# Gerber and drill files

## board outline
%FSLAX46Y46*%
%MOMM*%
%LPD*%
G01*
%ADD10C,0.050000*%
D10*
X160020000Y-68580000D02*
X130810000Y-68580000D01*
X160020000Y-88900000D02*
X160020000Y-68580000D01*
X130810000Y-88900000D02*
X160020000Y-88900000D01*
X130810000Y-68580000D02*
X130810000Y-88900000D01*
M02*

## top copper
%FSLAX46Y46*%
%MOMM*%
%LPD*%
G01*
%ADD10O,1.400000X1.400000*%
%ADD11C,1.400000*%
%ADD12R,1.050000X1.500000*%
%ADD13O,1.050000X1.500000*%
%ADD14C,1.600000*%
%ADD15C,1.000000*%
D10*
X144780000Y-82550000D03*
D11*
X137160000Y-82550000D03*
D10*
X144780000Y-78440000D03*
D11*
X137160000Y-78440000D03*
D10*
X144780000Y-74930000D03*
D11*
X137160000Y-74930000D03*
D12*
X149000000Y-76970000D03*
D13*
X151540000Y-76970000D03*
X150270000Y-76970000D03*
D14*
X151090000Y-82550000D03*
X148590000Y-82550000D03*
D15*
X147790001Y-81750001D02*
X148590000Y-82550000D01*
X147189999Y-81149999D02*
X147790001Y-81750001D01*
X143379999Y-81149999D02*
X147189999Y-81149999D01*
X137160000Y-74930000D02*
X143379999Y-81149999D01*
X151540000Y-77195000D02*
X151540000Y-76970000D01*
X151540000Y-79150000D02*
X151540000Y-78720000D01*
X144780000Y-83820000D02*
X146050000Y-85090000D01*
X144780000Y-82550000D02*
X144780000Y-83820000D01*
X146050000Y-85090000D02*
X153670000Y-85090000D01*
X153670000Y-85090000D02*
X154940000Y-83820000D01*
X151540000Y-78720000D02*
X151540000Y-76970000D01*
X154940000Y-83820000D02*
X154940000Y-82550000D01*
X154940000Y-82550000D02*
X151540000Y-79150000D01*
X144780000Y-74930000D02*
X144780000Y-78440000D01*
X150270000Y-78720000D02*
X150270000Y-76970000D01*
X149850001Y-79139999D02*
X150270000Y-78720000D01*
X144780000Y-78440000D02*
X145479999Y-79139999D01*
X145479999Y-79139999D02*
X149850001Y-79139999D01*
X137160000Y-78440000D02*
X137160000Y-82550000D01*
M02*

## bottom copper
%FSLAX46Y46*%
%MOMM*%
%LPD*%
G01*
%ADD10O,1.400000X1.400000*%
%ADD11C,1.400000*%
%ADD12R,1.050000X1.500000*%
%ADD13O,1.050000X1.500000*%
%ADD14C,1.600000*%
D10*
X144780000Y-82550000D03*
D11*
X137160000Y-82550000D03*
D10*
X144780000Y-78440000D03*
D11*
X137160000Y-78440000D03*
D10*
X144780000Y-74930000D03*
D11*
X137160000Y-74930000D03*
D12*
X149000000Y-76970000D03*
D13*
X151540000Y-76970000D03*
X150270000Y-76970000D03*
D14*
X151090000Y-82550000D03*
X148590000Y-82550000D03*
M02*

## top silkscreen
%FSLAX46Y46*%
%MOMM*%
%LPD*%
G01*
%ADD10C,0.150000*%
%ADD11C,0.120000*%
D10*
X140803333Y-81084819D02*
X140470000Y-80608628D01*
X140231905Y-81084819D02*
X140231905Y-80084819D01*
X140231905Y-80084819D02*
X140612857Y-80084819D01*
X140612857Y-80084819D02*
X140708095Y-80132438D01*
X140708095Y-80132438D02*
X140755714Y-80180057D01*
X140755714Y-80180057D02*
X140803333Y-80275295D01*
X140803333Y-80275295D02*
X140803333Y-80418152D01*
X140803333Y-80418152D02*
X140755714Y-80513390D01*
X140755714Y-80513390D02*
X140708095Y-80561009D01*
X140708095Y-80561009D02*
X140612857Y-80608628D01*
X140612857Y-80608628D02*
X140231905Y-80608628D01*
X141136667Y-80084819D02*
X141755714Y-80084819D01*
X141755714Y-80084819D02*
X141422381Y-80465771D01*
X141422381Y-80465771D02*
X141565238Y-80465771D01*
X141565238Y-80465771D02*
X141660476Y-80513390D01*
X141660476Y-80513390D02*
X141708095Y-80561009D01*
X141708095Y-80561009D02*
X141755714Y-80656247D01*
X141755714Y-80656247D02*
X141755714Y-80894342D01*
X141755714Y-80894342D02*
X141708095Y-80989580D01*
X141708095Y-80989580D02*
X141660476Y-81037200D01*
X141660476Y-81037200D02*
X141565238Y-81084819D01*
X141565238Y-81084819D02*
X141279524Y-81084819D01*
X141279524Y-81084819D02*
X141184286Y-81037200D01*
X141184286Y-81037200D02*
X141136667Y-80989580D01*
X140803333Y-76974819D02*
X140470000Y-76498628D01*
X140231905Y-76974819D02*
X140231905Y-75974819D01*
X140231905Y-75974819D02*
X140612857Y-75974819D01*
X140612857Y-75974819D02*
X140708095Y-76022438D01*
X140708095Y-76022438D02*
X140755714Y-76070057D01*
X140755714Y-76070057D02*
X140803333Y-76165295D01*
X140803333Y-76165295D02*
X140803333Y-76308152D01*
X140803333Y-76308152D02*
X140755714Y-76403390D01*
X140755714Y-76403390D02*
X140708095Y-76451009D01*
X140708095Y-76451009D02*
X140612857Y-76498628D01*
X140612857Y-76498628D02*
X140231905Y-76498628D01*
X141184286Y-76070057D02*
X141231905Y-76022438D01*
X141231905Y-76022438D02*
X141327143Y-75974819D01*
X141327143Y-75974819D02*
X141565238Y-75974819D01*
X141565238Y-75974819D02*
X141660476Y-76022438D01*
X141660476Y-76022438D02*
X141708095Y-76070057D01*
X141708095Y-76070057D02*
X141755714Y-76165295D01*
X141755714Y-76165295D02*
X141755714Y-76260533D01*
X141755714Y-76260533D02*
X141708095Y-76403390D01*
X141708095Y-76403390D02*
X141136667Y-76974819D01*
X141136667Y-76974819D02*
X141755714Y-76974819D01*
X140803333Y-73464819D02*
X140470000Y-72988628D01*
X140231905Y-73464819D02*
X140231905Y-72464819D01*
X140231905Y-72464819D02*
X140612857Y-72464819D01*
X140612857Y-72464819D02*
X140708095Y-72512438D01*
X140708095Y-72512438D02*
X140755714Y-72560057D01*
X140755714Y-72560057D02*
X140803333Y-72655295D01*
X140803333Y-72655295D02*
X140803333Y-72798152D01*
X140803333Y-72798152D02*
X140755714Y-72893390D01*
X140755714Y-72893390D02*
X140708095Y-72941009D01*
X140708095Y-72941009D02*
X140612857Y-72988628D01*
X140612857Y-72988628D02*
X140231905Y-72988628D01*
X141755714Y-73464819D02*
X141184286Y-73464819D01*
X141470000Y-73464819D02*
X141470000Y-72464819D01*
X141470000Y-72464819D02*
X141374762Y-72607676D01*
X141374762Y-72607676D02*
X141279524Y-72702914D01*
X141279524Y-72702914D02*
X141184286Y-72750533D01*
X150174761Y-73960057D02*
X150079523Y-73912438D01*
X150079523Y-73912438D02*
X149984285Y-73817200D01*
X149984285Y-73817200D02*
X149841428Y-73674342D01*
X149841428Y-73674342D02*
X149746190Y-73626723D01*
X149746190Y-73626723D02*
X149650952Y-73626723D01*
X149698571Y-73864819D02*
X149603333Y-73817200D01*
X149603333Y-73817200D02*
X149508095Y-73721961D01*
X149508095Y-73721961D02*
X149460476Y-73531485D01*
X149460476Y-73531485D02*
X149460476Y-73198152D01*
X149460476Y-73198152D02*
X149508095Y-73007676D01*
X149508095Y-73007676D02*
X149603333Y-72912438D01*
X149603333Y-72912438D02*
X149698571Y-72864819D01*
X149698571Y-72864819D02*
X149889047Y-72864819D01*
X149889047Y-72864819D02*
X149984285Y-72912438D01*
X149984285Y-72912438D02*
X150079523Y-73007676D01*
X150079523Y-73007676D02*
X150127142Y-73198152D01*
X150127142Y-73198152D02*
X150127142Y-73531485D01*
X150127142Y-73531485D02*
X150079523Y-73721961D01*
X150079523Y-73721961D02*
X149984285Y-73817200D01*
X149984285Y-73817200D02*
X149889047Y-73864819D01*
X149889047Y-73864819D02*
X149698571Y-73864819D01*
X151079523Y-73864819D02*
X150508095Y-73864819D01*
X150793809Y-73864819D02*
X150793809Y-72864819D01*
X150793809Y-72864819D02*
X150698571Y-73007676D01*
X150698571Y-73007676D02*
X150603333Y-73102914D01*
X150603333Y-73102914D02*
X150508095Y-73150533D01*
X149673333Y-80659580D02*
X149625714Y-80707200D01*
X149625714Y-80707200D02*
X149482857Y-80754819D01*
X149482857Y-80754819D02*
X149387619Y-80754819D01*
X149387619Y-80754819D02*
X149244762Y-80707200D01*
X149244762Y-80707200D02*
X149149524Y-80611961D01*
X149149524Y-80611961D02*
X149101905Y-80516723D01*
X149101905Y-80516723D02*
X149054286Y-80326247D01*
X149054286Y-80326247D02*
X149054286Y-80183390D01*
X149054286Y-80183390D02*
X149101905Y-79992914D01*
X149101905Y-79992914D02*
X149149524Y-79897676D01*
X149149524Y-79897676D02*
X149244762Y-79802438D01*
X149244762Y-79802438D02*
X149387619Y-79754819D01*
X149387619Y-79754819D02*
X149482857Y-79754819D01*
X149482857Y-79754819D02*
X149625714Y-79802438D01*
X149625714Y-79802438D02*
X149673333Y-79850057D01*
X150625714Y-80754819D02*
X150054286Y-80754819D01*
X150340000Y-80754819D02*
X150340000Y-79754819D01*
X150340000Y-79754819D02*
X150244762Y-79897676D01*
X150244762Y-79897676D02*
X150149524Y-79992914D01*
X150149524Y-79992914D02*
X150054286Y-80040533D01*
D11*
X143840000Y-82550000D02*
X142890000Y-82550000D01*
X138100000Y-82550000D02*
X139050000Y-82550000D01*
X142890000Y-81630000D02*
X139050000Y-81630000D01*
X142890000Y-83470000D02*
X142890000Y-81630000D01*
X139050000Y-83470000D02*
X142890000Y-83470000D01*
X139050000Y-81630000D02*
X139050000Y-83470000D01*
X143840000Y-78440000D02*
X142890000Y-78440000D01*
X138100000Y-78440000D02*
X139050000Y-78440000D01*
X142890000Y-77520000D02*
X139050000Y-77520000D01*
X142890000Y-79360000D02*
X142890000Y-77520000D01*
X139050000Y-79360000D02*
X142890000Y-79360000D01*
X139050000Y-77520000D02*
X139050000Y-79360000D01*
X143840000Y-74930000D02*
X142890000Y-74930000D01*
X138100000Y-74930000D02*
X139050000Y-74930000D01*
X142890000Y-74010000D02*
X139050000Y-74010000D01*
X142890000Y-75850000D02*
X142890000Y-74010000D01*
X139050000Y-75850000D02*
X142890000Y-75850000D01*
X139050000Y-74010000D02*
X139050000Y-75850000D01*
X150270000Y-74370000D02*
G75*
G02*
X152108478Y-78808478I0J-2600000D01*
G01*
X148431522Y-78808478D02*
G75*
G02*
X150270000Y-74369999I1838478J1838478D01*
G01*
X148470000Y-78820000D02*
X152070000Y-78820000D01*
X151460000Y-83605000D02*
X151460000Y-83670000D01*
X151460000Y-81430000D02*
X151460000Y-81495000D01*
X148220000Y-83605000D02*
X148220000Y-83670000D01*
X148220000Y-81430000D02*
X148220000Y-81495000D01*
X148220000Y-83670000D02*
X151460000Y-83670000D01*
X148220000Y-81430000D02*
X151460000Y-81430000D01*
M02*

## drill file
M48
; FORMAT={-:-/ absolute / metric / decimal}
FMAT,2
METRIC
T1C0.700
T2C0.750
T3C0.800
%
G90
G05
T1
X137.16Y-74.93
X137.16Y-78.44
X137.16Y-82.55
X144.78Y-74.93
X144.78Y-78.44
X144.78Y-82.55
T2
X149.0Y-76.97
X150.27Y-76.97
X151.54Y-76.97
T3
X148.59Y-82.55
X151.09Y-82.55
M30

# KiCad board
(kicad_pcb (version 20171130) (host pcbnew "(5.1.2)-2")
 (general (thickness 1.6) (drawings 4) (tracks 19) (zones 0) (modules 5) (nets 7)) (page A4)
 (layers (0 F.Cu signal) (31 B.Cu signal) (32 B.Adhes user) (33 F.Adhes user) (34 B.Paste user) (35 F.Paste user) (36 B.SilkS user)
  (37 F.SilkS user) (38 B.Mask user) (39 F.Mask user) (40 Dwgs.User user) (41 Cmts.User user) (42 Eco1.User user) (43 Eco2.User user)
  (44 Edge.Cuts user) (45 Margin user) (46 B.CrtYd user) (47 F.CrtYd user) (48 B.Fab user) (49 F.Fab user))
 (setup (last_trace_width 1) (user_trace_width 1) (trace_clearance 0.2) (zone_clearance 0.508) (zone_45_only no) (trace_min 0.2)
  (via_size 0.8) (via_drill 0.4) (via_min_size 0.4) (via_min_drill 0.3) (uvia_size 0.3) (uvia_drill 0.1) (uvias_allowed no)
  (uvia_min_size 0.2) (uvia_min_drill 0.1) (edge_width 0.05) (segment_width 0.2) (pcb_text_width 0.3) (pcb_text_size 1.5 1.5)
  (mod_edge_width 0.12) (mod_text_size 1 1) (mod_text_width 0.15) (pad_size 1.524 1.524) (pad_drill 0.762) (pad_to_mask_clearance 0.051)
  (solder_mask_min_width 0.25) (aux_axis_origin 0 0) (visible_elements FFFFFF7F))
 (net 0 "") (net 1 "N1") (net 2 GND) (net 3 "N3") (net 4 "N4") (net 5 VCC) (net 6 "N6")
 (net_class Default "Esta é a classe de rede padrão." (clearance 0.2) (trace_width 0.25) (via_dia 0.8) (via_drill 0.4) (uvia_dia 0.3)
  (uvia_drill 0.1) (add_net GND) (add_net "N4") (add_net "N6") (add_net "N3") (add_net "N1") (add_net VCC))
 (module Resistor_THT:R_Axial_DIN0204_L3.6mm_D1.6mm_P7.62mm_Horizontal (layer F.Cu) (at 137.16 82.55)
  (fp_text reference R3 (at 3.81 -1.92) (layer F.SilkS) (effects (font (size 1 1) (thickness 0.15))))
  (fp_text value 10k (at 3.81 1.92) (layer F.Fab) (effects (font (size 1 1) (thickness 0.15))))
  (fp_line (start 6.68 0) (end 5.73 0) (layer F.SilkS) (width 0.12))
  (fp_line (start 0.94 0) (end 1.89 0) (layer F.SilkS) (width 0.12))
  (fp_line (start 5.73 -0.92) (end 1.89 -0.92) (layer F.SilkS) (width 0.12))
  (fp_line (start 5.73 0.92) (end 5.73 -0.92) (layer F.SilkS) (width 0.12))
  (fp_line (start 1.89 0.92) (end 5.73 0.92) (layer F.SilkS) (width 0.12))
  (fp_line (start 1.89 -0.92) (end 1.89 0.92) (layer F.SilkS) (width 0.12))
  (pad 2 thru_hole oval (at 7.62 0) (size 1.4 1.4) (drill 0.7) (layers *.Cu *.Mask) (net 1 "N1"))
  (pad 1 thru_hole circle (at 0 0) (size 1.4 1.4) (drill 0.7) (layers *.Cu *.Mask) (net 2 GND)))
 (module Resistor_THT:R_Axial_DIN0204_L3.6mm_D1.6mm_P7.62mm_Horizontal (layer F.Cu) (at 137.16 78.44)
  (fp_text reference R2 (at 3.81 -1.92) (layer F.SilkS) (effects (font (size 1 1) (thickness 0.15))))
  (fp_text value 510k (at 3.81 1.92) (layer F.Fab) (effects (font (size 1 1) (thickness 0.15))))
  (fp_line (start 6.68 0) (end 5.73 0) (layer F.SilkS) (width 0.12))
  (fp_line (start 0.94 0) (end 1.89 0) (layer F.SilkS) (width 0.12))
  (fp_line (start 5.73 -0.92) (end 1.89 -0.92) (layer F.SilkS) (width 0.12))
  (fp_line (start 5.73 0.92) (end 5.73 -0.92) (layer F.SilkS) (width 0.12))
  (fp_line (start 1.89 0.92) (end 5.73 0.92) (layer F.SilkS) (width 0.12))
  (fp_line (start 1.89 -0.92) (end 1.89 0.92) (layer F.SilkS) (width 0.12))
  (pad 2 thru_hole oval (at 7.62 0) (size 1.4 1.4) (drill 0.7) (layers *.Cu *.Mask) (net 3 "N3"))
  (pad 1 thru_hole circle (at 0 0) (size 1.4 1.4) (drill 0.7) (layers *.Cu *.Mask) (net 2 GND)))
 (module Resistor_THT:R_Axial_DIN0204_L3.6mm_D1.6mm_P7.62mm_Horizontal (layer F.Cu) (at 137.16 74.93)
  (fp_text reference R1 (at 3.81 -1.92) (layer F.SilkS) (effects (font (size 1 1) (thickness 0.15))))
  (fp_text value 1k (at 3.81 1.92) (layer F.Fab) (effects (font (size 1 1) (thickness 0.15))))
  (fp_line (start 6.68 0) (end 5.73 0) (layer F.SilkS) (width 0.12))
  (fp_line (start 0.94 0) (end 1.89 0) (layer F.SilkS) (width 0.12))
  (fp_line (start 5.73 -0.92) (end 1.89 -0.92) (layer F.SilkS) (width 0.12))
  (fp_line (start 5.73 0.92) (end 5.73 -0.92) (layer F.SilkS) (width 0.12))
  (fp_line (start 1.89 0.92) (end 5.73 0.92) (layer F.SilkS) (width 0.12))
  (fp_line (start 1.89 -0.92) (end 1.89 0.92) (layer F.SilkS) (width 0.12))
  (pad 2 thru_hole oval (at 7.62 0) (size 1.4 1.4) (drill 0.7) (layers *.Cu *.Mask) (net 3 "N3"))
  (pad 1 thru_hole circle (at 0 0) (size 1.4 1.4) (drill 0.7) (layers *.Cu *.Mask) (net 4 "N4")))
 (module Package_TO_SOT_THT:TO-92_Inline (layer F.Cu) (at 149 76.97)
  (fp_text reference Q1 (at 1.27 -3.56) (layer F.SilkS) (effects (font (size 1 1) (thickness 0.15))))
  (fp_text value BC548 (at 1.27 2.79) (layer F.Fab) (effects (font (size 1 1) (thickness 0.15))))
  (fp_arc (start 1.27 0) (end 1.27 -2.6) (angle 135) (layer F.SilkS) (width 0.12))
  (fp_arc (start 1.27 0) (end 1.27 -2.6) (angle -135) (layer F.SilkS) (width 0.12))
  (fp_line (start -0.53 1.85) (end 3.07 1.85) (layer F.SilkS) (width 0.12))
  (pad 1 thru_hole rect (at 0 0) (size 1.05 1.5) (drill 0.75) (layers *.Cu *.Mask) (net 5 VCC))
  (pad 3 thru_hole oval (at 2.54 0) (size 1.05 1.5) (drill 0.75) (layers *.Cu *.Mask) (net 1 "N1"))
  (pad 2 thru_hole oval (at 1.27 0) (size 1.05 1.5) (drill 0.75) (layers *.Cu *.Mask) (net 3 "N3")))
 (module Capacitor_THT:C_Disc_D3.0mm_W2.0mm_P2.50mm (layer F.Cu) (at 148.59 82.55)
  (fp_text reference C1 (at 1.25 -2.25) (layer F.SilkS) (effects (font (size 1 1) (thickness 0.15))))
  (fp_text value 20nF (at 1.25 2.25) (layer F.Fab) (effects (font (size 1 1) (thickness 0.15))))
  (fp_line (start 2.87 1.055) (end 2.87 1.12) (layer F.SilkS) (width 0.12))
  (fp_line (start 2.87 -1.12) (end 2.87 -1.055) (layer F.SilkS) (width 0.12))
  (fp_line (start -0.37 1.055) (end -0.37 1.12) (layer F.SilkS) (width 0.12))
  (fp_line (start -0.37 -1.12) (end -0.37 -1.055) (layer F.SilkS) (width 0.12))
  (fp_line (start -0.37 1.12) (end 2.87 1.12) (layer F.SilkS) (width 0.12))
  (fp_line (start -0.37 -1.12) (end 2.87 -1.12) (layer F.SilkS) (width 0.12))
  (pad 2 thru_hole circle (at 2.5 0) (size 1.6 1.6) (drill 0.8) (layers *.Cu *.Mask) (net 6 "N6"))
  (pad 1 thru_hole circle (at 0 0) (size 1.6 1.6) (drill 0.8) (layers *.Cu *.Mask) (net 4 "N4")))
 (gr_line (start 160.02 68.58) (end 130.81 68.58) (layer Edge.Cuts) (width 0.05))
 (gr_line (start 160.02 88.9) (end 160.02 68.58) (layer Edge.Cuts) (width 0.05))
 (gr_line (start 130.81 88.9) (end 160.02 88.9) (layer Edge.Cuts) (width 0.05))
 (gr_line (start 130.81 68.58) (end 130.81 88.9) (layer Edge.Cuts) (width 0.05))
 (segment (start 147.790001 81.750001) (end 148.59 82.55) (width 1) (layer F.Cu) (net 4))
 (segment (start 147.189999 81.149999) (end 147.790001 81.750001) (width 1) (layer F.Cu) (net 4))
 (segment (start 143.379999 81.149999) (end 147.189999 81.149999) (width 1) (layer F.Cu) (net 4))
 (segment (start 137.16 74.93) (end 143.379999 81.149999) (width 1) (layer F.Cu) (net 4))
 (segment (start 151.54 77.195) (end 151.54 76.97) (width 1) (layer F.Cu) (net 1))
 (segment (start 151.54 79.15) (end 151.54 78.72) (width 1) (layer F.Cu) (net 1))
 (segment (start 144.78 83.82) (end 146.05 85.09) (width 1) (layer F.Cu) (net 1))
 (segment (start 144.78 82.55) (end 144.78 83.82) (width 1) (layer F.Cu) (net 1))
 (segment (start 146.05 85.09) (end 153.67 85.09) (width 1) (layer F.Cu) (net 1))
 (segment (start 153.67 85.09) (end 154.94 83.82) (width 1) (layer F.Cu) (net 1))
 (segment (start 151.54 78.72) (end 151.54 76.97) (width 1) (layer F.Cu) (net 1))
 (segment (start 154.94 83.82) (end 154.94 82.55) (width 1) (layer F.Cu) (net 1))
 (segment (start 154.94 82.55) (end 151.54 79.15) (width 1) (layer F.Cu) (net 1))
 (segment (start 144.78 74.93) (end 144.78 78.44) (width 1) (layer F.Cu) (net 3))
 (segment (start 150.27 78.72) (end 150.27 76.97) (width 1) (layer F.Cu) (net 3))
 (segment (start 149.850001 79.139999) (end 150.27 78.72) (width 1) (layer F.Cu) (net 3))
 (segment (start 144.78 78.44) (end 145.479999 79.139999) (width 1) (layer F.Cu) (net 3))
 (segment (start 145.479999 79.139999) (end 149.850001 79.139999) (width 1) (layer F.Cu) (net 3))
 (segment (start 137.16 78.44) (end 137.16 82.55) (width 1) (layer F.Cu) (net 2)))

